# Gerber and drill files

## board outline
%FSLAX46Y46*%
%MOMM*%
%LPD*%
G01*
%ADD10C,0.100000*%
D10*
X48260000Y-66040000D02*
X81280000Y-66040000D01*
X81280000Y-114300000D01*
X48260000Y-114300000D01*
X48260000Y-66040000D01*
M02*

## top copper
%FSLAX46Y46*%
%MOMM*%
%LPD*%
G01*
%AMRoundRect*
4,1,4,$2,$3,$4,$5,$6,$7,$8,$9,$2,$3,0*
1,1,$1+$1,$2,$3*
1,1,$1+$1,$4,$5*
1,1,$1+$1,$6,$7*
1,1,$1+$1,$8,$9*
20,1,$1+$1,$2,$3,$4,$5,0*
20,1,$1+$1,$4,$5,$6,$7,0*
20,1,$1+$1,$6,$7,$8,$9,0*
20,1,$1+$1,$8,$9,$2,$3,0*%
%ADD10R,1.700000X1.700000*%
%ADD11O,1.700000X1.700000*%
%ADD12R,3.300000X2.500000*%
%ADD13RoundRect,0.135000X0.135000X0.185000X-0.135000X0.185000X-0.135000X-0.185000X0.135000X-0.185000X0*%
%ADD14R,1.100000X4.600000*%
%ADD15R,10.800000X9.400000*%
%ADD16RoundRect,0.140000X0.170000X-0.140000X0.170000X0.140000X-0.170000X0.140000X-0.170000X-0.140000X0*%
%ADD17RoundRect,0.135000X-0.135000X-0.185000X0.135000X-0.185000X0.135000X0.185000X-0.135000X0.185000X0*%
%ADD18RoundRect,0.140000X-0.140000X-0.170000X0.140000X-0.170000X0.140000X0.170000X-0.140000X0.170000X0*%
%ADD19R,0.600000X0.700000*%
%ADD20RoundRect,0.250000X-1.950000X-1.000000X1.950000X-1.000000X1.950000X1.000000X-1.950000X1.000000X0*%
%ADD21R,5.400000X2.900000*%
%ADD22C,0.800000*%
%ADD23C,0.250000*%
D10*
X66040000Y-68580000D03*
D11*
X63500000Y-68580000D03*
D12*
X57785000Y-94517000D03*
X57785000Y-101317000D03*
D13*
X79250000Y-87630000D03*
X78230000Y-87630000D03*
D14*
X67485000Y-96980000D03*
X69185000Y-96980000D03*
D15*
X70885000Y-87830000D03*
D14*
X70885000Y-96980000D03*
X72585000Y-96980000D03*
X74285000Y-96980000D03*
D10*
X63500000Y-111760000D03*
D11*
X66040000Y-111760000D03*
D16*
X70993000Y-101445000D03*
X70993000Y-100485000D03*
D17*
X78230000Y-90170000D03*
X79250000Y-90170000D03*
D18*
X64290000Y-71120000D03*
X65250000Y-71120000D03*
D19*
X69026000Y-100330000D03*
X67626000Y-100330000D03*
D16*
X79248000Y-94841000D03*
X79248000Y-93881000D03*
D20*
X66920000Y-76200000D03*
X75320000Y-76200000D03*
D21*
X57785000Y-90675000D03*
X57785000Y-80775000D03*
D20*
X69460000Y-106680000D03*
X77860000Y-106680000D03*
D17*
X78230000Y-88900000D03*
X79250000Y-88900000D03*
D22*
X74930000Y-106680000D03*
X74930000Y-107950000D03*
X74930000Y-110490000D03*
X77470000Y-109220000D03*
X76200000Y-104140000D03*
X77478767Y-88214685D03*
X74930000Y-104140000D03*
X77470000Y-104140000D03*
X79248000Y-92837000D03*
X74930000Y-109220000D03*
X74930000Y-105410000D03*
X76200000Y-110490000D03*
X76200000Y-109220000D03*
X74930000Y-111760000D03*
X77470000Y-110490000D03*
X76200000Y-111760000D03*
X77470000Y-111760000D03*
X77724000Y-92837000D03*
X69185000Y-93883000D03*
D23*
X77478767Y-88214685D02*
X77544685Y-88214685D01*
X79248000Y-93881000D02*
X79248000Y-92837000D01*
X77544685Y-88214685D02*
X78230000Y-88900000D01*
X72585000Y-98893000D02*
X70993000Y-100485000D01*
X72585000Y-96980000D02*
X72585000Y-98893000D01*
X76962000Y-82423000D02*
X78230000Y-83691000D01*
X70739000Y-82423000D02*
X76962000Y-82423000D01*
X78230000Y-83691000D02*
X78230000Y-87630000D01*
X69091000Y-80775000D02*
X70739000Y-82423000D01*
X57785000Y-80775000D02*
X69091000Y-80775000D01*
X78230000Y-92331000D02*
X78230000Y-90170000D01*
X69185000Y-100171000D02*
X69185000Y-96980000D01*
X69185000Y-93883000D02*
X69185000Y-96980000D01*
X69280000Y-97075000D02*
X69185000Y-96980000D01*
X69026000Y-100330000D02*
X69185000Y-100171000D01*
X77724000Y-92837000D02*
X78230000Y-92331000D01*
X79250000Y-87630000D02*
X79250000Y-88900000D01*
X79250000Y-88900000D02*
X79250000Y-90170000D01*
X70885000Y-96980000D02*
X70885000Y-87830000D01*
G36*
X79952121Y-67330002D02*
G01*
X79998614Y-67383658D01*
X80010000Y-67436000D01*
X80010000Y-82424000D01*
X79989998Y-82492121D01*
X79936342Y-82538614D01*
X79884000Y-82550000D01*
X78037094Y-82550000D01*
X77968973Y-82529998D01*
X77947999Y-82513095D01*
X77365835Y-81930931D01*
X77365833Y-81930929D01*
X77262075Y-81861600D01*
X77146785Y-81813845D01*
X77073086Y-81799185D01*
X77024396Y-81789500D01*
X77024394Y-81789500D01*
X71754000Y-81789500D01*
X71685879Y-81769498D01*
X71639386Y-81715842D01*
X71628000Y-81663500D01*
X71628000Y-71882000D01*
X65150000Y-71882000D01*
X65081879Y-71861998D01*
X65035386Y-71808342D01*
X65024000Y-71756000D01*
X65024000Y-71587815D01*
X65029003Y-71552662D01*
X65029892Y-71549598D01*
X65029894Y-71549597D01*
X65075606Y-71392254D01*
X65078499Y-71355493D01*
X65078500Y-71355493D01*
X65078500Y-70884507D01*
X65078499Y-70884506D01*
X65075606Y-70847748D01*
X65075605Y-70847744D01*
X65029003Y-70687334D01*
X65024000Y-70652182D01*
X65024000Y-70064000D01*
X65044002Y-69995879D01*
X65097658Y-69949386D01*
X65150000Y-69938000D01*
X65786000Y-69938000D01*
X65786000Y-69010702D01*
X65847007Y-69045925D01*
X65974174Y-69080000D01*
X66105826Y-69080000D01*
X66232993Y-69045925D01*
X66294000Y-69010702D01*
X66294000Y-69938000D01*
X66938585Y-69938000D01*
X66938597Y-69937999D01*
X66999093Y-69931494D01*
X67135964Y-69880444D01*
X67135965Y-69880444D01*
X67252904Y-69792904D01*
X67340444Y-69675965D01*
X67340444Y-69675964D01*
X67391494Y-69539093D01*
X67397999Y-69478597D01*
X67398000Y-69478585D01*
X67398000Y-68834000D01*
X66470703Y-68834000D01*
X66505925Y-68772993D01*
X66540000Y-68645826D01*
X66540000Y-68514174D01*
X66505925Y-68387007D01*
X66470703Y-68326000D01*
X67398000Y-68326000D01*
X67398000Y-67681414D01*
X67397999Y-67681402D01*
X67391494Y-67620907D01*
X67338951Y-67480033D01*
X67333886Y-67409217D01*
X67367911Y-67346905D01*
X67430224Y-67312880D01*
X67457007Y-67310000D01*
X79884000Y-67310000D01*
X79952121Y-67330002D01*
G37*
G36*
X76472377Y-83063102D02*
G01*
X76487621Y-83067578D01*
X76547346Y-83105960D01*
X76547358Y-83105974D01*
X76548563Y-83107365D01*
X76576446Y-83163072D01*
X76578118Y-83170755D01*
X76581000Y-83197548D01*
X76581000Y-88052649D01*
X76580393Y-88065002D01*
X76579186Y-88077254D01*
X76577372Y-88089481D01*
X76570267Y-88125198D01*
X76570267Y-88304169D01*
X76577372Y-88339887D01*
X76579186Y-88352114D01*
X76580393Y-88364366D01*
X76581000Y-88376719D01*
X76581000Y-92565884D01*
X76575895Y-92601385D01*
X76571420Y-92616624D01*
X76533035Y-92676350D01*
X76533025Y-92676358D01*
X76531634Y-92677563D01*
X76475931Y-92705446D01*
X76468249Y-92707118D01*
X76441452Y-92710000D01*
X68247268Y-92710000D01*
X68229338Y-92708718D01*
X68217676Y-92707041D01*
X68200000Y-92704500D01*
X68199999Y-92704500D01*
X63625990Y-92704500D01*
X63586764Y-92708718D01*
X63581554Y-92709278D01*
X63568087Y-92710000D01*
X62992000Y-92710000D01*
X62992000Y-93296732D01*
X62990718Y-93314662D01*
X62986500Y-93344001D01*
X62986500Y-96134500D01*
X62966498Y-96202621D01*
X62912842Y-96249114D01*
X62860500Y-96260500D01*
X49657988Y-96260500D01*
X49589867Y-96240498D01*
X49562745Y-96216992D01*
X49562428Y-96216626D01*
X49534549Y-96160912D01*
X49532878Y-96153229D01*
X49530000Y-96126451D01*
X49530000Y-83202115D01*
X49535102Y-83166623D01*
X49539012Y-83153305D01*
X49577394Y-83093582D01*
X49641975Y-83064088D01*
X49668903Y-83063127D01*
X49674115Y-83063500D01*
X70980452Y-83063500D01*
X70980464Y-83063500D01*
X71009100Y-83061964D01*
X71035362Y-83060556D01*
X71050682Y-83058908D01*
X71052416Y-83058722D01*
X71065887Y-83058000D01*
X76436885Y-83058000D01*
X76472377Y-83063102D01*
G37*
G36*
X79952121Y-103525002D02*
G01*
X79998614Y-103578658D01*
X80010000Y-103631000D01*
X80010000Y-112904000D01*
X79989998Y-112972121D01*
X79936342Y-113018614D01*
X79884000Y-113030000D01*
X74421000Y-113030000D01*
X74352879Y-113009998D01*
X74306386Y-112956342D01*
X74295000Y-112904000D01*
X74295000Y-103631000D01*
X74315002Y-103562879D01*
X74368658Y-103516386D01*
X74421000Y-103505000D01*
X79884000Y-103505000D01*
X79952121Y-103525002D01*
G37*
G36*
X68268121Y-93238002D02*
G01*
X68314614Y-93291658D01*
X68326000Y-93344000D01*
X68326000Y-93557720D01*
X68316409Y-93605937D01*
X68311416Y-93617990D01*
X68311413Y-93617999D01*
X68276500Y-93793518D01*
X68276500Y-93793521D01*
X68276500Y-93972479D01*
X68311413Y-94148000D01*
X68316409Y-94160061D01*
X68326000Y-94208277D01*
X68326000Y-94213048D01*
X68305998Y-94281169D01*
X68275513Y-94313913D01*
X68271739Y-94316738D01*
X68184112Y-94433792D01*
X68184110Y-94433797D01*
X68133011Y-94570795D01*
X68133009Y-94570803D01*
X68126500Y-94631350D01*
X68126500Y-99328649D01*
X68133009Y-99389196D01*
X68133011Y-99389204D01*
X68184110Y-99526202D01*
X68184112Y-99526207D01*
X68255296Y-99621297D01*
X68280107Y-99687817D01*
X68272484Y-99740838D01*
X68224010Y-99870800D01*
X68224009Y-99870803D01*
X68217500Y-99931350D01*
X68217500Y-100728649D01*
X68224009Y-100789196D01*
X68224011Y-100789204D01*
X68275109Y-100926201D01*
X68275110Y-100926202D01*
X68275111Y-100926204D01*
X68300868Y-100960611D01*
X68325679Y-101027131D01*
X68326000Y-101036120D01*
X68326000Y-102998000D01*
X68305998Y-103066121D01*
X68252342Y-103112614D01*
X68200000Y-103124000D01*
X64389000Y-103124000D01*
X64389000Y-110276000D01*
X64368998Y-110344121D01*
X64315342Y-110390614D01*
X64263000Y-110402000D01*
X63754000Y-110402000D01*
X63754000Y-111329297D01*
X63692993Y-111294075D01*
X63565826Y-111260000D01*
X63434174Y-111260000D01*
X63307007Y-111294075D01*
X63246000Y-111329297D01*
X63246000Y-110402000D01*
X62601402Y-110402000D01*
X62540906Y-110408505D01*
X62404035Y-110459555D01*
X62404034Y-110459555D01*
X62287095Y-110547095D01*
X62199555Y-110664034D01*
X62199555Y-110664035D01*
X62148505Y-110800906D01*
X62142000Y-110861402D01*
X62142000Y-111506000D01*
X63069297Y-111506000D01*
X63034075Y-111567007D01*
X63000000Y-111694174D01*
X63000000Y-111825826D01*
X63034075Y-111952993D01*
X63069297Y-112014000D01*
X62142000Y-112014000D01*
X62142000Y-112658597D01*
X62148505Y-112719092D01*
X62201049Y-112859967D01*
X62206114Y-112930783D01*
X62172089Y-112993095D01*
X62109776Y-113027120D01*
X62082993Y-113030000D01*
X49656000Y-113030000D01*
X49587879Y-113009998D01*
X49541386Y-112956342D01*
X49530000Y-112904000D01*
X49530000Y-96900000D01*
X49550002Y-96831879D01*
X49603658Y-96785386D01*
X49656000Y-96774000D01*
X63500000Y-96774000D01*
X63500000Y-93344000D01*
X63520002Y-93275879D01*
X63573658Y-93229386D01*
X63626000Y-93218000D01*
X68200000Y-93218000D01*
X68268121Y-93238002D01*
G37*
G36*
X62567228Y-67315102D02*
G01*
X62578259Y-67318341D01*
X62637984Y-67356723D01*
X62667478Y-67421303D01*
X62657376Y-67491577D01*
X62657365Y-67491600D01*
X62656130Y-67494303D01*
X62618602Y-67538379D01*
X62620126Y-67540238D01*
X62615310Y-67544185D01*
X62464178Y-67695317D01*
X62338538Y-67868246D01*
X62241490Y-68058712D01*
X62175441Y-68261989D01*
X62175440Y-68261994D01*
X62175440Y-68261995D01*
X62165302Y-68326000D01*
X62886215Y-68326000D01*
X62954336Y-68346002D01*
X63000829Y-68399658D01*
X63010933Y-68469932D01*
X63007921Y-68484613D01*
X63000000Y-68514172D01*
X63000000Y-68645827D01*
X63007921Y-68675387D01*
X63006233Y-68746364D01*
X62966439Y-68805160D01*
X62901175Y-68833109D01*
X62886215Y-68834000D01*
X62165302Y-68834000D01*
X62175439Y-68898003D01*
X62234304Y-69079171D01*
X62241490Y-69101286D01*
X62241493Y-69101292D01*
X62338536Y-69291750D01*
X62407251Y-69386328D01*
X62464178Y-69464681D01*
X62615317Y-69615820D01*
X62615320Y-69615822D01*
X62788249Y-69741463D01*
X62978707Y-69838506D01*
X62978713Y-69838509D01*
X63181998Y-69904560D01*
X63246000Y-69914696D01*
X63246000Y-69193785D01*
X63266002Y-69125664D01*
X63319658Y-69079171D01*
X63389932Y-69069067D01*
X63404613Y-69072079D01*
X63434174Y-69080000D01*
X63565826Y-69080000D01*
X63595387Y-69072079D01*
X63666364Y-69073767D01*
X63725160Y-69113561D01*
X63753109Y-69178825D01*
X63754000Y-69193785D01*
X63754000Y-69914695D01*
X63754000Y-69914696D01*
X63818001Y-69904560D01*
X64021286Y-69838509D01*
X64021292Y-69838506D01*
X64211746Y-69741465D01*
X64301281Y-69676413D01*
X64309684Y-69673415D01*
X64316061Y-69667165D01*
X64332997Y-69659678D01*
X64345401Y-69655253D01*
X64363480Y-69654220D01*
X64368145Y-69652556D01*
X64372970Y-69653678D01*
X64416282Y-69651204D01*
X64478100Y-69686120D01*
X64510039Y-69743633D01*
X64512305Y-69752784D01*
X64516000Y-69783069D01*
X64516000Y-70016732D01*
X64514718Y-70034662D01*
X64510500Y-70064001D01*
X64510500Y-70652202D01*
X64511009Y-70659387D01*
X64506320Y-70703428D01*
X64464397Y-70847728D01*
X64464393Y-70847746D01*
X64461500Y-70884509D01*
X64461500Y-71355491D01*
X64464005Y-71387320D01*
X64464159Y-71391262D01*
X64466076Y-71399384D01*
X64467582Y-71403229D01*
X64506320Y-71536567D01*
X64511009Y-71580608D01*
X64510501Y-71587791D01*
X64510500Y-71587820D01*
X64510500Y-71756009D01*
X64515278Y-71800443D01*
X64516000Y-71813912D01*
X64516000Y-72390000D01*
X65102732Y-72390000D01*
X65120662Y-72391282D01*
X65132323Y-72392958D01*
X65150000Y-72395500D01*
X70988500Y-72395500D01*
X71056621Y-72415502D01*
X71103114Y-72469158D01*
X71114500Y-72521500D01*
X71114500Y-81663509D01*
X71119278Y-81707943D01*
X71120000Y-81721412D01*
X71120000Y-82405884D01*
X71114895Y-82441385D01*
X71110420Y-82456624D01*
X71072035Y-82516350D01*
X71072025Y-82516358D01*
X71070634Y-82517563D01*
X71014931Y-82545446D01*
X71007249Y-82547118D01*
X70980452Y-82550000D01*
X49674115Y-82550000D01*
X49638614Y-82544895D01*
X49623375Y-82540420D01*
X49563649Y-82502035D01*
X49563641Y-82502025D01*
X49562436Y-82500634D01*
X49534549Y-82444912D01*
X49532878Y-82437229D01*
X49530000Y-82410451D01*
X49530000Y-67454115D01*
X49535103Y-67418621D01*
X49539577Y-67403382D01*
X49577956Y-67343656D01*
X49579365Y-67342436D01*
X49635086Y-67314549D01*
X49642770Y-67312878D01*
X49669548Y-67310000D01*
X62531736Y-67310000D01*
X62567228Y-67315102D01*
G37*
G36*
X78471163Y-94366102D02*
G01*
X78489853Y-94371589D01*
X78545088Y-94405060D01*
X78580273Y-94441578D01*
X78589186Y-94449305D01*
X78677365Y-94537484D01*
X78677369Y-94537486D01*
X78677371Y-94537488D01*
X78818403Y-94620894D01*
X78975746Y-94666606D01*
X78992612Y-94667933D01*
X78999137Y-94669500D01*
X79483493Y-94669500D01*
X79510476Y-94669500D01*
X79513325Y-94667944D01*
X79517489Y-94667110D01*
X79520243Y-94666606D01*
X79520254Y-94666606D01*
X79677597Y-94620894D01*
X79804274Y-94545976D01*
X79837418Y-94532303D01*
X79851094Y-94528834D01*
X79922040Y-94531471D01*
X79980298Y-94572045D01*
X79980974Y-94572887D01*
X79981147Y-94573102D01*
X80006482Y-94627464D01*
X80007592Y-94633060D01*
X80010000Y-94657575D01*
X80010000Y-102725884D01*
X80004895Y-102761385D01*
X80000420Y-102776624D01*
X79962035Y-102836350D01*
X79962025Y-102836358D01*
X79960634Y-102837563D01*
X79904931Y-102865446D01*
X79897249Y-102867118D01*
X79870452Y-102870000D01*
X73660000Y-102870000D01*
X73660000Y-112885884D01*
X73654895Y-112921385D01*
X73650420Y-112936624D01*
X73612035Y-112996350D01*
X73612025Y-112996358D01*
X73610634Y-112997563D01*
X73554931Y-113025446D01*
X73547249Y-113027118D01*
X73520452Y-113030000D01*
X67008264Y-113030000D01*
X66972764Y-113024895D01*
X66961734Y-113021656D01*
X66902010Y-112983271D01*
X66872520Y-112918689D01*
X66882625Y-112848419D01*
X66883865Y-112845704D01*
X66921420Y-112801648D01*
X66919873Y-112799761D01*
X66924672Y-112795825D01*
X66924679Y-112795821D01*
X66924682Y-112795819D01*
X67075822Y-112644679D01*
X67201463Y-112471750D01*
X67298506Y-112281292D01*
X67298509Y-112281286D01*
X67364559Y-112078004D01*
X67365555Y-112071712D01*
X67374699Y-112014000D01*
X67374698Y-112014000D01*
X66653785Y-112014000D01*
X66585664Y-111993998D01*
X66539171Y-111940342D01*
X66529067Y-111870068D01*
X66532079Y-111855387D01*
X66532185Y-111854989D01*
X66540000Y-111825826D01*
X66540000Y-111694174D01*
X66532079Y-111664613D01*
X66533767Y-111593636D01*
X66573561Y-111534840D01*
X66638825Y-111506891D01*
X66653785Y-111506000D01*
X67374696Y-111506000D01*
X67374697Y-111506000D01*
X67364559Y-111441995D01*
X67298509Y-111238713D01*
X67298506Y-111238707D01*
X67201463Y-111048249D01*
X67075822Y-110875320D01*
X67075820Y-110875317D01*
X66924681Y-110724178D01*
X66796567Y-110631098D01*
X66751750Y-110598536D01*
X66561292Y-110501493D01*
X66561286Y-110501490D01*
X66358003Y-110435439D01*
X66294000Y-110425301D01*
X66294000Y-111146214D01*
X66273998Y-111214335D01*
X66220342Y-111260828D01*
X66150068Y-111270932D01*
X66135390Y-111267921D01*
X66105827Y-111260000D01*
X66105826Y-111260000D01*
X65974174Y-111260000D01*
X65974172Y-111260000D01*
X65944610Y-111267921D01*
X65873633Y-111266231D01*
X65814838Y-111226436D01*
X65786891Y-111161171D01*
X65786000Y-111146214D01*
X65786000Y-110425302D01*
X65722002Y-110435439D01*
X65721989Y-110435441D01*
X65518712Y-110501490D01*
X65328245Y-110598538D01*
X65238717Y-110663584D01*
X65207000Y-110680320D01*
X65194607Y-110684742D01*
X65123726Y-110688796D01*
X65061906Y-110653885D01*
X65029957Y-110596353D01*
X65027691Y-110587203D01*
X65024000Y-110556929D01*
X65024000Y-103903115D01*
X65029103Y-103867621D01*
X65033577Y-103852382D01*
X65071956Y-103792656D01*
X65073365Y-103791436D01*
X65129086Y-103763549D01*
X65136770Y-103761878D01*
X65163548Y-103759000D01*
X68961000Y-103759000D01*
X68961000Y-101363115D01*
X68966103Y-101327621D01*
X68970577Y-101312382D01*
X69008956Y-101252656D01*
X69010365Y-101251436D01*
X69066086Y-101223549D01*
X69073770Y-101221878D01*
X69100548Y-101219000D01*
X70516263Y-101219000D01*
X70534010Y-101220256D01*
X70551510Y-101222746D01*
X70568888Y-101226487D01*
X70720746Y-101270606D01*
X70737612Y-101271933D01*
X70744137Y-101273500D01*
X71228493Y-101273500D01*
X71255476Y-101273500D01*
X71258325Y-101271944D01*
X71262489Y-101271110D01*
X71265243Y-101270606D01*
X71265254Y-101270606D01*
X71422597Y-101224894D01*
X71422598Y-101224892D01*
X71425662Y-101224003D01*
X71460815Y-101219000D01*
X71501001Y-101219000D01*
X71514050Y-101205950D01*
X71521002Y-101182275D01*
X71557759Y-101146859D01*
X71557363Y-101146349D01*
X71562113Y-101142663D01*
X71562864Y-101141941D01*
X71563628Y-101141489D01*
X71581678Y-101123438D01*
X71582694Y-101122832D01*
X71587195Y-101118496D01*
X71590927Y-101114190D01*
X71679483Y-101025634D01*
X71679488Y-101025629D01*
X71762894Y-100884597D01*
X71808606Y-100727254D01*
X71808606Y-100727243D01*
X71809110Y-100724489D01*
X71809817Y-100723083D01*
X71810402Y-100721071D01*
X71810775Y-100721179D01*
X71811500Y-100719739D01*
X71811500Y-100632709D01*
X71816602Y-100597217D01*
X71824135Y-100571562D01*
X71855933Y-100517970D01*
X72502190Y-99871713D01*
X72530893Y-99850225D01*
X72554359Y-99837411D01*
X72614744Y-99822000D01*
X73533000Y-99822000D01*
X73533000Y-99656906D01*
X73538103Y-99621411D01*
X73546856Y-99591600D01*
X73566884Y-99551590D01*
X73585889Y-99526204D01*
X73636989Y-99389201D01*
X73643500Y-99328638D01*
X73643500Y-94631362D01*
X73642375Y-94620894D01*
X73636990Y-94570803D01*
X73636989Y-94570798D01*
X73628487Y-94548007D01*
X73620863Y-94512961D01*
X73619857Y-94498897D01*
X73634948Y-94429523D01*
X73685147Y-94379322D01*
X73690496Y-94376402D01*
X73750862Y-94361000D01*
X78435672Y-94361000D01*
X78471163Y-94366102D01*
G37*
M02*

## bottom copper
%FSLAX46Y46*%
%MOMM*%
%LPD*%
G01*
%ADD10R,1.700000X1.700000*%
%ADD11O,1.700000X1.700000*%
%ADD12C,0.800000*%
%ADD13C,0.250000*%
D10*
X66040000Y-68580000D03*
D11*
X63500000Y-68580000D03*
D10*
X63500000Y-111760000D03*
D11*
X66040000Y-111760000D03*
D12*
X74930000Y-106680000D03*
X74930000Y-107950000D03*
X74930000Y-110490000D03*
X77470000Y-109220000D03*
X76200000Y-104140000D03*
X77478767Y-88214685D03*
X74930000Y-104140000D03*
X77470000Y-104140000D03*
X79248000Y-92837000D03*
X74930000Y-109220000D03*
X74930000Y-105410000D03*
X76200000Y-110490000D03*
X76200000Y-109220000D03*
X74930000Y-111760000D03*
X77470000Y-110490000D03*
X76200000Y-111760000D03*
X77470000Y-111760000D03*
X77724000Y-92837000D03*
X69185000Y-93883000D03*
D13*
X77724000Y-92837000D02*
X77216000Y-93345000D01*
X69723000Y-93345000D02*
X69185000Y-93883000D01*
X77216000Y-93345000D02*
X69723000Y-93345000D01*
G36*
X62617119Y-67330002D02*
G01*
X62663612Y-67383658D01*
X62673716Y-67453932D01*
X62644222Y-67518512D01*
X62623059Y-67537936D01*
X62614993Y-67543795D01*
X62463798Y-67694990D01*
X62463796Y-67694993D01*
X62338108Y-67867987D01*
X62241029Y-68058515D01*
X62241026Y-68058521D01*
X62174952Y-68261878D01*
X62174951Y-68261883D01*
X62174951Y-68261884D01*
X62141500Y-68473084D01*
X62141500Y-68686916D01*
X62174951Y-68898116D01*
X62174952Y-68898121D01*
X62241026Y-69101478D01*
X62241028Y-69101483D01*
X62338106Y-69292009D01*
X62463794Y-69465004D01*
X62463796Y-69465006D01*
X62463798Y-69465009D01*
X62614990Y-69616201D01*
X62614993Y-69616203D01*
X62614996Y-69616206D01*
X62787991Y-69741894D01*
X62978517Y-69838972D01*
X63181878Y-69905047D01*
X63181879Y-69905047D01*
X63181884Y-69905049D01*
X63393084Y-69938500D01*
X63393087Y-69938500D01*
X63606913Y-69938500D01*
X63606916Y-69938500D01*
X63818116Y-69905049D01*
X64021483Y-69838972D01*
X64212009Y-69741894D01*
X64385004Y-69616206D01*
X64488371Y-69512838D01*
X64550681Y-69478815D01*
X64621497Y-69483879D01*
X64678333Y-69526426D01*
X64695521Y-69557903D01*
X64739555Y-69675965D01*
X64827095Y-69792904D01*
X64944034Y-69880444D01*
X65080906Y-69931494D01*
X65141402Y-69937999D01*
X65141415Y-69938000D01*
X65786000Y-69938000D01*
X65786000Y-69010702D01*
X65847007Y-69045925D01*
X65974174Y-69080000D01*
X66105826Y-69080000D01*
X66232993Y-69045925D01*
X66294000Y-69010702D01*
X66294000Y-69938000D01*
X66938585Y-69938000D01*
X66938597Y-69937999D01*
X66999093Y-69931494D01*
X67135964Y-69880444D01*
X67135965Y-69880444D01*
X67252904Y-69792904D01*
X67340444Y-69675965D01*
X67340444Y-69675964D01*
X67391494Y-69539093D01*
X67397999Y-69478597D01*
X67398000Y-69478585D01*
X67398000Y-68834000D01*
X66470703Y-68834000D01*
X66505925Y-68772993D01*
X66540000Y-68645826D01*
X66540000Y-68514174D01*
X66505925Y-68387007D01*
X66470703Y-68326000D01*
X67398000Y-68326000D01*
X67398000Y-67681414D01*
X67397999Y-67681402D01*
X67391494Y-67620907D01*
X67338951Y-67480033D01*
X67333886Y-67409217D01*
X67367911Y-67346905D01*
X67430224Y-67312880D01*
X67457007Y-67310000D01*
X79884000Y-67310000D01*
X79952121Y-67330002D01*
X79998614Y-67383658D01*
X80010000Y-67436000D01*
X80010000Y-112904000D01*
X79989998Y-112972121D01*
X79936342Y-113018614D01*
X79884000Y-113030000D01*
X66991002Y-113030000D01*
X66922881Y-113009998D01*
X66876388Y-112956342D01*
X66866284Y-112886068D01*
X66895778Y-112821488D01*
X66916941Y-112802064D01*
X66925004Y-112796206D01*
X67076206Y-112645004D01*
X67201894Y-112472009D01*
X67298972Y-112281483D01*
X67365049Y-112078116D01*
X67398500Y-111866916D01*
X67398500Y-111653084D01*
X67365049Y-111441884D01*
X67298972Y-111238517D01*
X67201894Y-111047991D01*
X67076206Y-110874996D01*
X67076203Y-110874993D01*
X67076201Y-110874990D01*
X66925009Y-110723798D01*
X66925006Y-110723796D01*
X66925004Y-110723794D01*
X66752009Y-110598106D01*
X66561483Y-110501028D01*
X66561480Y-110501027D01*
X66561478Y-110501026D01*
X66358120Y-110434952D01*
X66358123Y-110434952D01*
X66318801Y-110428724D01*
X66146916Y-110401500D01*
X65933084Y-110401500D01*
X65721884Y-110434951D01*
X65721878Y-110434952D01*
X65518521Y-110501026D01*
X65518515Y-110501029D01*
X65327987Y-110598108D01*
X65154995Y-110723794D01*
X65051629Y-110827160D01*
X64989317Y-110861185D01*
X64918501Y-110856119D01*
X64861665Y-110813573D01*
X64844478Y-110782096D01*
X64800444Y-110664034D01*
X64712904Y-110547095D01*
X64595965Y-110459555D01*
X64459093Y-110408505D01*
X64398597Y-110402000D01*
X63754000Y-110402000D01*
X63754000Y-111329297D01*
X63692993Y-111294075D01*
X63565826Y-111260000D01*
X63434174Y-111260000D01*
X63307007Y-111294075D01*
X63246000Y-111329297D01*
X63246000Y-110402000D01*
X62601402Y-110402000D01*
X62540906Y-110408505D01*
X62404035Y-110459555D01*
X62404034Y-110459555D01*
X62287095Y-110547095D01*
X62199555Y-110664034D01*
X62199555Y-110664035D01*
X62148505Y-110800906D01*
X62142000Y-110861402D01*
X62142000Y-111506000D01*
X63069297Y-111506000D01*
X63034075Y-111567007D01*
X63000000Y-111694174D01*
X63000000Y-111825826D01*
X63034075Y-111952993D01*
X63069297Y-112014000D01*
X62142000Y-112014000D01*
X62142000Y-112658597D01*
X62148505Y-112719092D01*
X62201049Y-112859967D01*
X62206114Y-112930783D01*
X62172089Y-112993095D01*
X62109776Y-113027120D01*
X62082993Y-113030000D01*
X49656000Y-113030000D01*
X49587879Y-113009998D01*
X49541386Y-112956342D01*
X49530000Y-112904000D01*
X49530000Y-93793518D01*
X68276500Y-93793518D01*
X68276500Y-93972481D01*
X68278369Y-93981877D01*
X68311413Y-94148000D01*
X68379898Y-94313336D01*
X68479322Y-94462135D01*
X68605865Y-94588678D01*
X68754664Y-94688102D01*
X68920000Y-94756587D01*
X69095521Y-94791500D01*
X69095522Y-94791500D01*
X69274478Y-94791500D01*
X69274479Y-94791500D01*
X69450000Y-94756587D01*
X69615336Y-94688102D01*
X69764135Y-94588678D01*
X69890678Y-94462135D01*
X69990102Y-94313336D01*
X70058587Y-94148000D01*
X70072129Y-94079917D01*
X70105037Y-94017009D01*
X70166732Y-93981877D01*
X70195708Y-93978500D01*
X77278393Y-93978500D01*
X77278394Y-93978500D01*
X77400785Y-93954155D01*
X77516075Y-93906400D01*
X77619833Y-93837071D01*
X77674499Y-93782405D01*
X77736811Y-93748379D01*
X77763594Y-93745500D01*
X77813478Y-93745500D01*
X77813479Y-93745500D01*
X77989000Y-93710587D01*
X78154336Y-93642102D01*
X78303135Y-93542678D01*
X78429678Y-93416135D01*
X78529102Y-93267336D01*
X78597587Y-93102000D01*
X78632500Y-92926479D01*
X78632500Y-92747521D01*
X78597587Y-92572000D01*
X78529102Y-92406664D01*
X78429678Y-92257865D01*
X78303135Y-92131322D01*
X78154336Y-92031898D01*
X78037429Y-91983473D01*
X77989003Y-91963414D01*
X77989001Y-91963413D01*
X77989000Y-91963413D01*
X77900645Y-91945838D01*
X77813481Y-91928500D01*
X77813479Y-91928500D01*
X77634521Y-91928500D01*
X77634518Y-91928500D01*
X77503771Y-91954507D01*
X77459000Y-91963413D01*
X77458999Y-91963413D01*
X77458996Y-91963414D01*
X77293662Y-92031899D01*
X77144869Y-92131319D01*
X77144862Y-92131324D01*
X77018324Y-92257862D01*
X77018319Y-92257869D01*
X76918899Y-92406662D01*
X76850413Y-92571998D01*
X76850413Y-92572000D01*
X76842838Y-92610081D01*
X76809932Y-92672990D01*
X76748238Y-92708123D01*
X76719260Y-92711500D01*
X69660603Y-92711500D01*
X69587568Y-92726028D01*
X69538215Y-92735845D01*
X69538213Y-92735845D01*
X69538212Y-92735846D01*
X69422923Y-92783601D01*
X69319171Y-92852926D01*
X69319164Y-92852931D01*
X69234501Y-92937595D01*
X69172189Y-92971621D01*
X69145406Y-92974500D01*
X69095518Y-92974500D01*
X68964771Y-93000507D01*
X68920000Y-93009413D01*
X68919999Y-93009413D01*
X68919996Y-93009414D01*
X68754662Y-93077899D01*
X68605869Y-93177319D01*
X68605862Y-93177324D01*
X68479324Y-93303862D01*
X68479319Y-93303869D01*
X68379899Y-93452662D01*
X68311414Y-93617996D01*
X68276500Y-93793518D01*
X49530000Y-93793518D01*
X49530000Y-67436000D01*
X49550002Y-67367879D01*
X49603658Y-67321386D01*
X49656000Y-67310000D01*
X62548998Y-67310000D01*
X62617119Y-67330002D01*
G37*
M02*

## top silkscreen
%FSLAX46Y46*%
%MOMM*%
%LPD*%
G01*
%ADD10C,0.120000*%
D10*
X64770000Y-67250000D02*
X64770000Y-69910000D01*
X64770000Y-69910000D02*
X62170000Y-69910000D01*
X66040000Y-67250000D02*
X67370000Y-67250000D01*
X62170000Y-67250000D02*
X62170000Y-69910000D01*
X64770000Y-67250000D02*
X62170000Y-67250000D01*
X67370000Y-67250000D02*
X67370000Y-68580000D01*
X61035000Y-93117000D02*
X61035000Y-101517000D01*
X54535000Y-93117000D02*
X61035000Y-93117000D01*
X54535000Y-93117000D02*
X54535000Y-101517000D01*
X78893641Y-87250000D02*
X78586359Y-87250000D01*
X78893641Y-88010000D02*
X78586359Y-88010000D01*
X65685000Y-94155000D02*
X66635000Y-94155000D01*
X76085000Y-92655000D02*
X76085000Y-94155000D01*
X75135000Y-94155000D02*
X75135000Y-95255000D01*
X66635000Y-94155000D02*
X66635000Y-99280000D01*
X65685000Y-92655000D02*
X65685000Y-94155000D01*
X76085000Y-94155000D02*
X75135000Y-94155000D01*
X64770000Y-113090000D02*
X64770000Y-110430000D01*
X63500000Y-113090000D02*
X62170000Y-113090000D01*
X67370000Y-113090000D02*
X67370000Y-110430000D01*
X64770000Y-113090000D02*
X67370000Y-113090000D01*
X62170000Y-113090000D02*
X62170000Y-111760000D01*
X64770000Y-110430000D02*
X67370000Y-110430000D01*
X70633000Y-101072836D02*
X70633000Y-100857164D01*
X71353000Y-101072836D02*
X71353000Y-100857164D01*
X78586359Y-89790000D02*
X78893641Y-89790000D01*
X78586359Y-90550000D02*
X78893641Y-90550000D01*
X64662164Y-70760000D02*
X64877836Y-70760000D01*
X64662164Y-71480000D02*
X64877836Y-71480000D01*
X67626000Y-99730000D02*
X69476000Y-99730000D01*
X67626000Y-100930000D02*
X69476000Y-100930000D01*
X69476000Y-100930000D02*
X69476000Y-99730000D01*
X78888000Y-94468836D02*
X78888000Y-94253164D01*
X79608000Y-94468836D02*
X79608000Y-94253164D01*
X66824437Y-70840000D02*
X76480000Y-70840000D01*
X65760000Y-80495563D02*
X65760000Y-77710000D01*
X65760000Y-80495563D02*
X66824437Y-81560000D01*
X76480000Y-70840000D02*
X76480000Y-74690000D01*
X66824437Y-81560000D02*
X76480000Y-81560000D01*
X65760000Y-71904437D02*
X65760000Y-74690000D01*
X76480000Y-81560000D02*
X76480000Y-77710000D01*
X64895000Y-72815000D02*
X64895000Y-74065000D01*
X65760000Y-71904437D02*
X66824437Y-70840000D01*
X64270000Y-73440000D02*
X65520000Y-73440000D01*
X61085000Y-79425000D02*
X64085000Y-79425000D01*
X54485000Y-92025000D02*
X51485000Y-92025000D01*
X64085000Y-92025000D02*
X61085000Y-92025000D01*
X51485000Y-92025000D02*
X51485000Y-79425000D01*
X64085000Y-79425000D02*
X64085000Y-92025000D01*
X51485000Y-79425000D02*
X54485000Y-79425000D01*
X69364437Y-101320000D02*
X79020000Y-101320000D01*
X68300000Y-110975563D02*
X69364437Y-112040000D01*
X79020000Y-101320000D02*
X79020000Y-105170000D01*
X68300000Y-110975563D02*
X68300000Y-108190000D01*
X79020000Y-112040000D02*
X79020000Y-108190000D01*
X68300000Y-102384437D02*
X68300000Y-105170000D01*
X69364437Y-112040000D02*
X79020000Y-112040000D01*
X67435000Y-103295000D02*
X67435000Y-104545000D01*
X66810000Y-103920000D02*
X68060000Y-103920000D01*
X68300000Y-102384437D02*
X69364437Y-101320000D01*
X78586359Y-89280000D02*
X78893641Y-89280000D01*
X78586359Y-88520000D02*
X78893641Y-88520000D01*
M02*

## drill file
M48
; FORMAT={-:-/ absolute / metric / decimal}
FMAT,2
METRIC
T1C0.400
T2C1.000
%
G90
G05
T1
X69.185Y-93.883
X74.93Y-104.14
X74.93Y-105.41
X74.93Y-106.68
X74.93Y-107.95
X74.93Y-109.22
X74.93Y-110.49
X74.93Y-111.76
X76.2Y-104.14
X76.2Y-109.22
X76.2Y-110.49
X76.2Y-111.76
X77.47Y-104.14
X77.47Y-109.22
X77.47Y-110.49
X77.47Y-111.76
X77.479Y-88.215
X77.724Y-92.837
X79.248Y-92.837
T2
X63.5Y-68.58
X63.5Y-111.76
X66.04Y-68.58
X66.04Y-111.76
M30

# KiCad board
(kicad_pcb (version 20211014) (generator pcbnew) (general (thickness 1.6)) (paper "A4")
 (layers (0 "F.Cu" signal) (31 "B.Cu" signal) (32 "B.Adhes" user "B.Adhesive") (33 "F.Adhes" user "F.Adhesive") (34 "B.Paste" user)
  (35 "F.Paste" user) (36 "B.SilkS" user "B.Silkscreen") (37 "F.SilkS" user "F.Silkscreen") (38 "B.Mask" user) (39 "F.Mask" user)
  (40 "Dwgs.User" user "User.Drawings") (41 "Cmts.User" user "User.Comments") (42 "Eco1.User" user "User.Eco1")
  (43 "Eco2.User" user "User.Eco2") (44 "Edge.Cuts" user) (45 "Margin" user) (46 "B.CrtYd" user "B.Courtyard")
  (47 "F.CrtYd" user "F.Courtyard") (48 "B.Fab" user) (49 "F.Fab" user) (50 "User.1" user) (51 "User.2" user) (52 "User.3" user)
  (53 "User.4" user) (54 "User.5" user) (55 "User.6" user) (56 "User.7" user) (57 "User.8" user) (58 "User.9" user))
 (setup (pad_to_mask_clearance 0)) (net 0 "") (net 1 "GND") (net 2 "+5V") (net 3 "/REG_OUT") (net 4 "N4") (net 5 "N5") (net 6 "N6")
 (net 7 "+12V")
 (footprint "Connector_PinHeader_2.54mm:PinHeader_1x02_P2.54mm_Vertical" (layer "F.Cu") (at 66.04 68.58 -90)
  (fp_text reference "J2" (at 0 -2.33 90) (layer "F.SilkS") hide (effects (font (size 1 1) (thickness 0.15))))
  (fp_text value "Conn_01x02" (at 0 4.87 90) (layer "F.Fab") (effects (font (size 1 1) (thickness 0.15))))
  (fp_line (start -1.33 1.27) (end 1.33 1.27) (layer "F.SilkS") (width 0.12))
  (fp_line (start 1.33 1.27) (end 1.33 3.87) (layer "F.SilkS") (width 0.12))
  (fp_line (start -1.33 0) (end -1.33 -1.33) (layer "F.SilkS") (width 0.12))
  (fp_line (start -1.33 3.87) (end 1.33 3.87) (layer "F.SilkS") (width 0.12))
  (fp_line (start -1.33 1.27) (end -1.33 3.87) (layer "F.SilkS") (width 0.12))
  (fp_line (start -1.33 -1.33) (end 0 -1.33) (layer "F.SilkS") (width 0.12))
  (pad "1" thru_hole rect (at 0 0 270) (size 1.7 1.7) (drill 1) (layers *.Cu *.Mask) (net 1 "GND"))
  (pad "2" thru_hole oval (at 0 2.54 270) (size 1.7 1.7) (drill 1) (layers *.Cu *.Mask) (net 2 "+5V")))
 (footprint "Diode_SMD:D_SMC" (layer "F.Cu") (at 57.785 97.917 -90)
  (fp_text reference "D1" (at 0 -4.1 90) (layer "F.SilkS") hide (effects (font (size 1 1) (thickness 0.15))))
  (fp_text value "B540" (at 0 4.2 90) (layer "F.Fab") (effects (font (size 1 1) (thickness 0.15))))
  (fp_line (start -4.8 -3.25) (end 3.6 -3.25) (layer "F.SilkS") (width 0.12))
  (fp_line (start -4.8 3.25) (end -4.8 -3.25) (layer "F.SilkS") (width 0.12))
  (fp_line (start -4.8 3.25) (end 3.6 3.25) (layer "F.SilkS") (width 0.12))
  (pad "1" smd rect (at -3.4 0) (size 3.3 2.5) (layers "F.Cu" "F.Paste" "F.Mask") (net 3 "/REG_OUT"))
  (pad "2" smd rect (at 3.4 0) (size 3.3 2.5) (layers "F.Cu" "F.Paste" "F.Mask") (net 1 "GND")))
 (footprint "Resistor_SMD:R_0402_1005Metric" (layer "F.Cu") (at 78.74 87.63 180)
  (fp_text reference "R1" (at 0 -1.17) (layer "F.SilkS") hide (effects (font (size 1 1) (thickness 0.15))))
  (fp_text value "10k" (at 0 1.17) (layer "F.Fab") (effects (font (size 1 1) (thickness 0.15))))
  (fp_line (start -0.153641 0.38) (end 0.153641 0.38) (layer "F.SilkS") (width 0.12))
  (fp_line (start -0.153641 -0.38) (end 0.153641 -0.38) (layer "F.SilkS") (width 0.12))
  (pad "1" smd roundrect (at -0.51 0 180) (size 0.54 0.64) (layers "F.Cu" "F.Paste" "F.Mask") (roundrect_rratio 0.25) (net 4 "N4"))
  (pad "2" smd roundrect (at 0.51 0 180) (size 0.54 0.64) (layers "F.Cu" "F.Paste" "F.Mask") (roundrect_rratio 0.25) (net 2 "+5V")))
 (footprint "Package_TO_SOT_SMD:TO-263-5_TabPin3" (layer "F.Cu") (at 70.885 91.205 90)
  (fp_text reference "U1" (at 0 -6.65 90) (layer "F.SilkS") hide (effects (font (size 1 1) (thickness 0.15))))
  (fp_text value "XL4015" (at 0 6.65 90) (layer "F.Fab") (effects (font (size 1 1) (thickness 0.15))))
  (fp_line (start -2.95 -5.2) (end -2.95 -4.25) (layer "F.SilkS") (width 0.12))
  (fp_line (start -1.45 5.2) (end -2.95 5.2) (layer "F.SilkS") (width 0.12))
  (fp_line (start -2.95 4.25) (end -4.05 4.25) (layer "F.SilkS") (width 0.12))
  (fp_line (start -2.95 -4.25) (end -8.075 -4.25) (layer "F.SilkS") (width 0.12))
  (fp_line (start -1.45 -5.2) (end -2.95 -5.2) (layer "F.SilkS") (width 0.12))
  (fp_line (start -2.95 5.2) (end -2.95 4.25) (layer "F.SilkS") (width 0.12))
  (pad "" smd rect (at 5.8 2.775 90) (size 4.55 5.25) (layers "F.Paste"))
  (pad "" smd rect (at 0.95 -2.775 90) (size 4.55 5.25) (layers "F.Paste"))
  (pad "" smd rect (at 5.8 -2.775 90) (size 4.55 5.25) (layers "F.Paste"))
  (pad "" smd rect (at 0.95 2.775 90) (size 4.55 5.25) (layers "F.Paste"))
  (pad "1" smd rect (at -5.775 -3.4 90) (size 4.6 1.1) (layers "F.Cu" "F.Paste" "F.Mask") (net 1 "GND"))
  (pad "2" smd rect (at -5.775 -1.7 90) (size 4.6 1.1) (layers "F.Cu" "F.Paste" "F.Mask") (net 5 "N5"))
  (pad "3" smd rect (at 3.375 0 90) (size 9.4 10.8) (layers "F.Cu" "F.Mask") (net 3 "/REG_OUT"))
  (pad "3" smd rect (at -5.775 0 90) (size 4.6 1.1) (layers "F.Cu" "F.Paste" "F.Mask") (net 3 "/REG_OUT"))
  (pad "4" smd rect (at -5.775 1.7 90) (size 4.6 1.1) (layers "F.Cu" "F.Paste" "F.Mask") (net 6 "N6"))
  (pad "5" smd rect (at -5.775 3.4 90) (size 4.6 1.1) (layers "F.Cu" "F.Paste" "F.Mask") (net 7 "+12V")))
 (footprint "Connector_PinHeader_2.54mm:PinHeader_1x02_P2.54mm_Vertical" (layer "F.Cu") (at 63.5 111.76 90)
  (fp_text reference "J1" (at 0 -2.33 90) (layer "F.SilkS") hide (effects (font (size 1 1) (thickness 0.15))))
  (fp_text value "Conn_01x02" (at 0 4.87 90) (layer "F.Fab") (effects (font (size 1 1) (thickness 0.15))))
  (fp_line (start -1.33 1.27) (end 1.33 1.27) (layer "F.SilkS") (width 0.12))
  (fp_line (start -1.33 0) (end -1.33 -1.33) (layer "F.SilkS") (width 0.12))
  (fp_line (start -1.33 3.87) (end 1.33 3.87) (layer "F.SilkS") (width 0.12))
  (fp_line (start -1.33 1.27) (end -1.33 3.87) (layer "F.SilkS") (width 0.12))
  (fp_line (start -1.33 -1.33) (end 0 -1.33) (layer "F.SilkS") (width 0.12))
  (fp_line (start 1.33 1.27) (end 1.33 3.87) (layer "F.SilkS") (width 0.12))
  (pad "1" thru_hole rect (at 0 0 90) (size 1.7 1.7) (drill 1) (layers *.Cu *.Mask) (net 1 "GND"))
  (pad "2" thru_hole oval (at 0 2.54 90) (size 1.7 1.7) (drill 1) (layers *.Cu *.Mask) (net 7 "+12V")))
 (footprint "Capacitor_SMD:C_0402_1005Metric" (layer "F.Cu") (at 70.993 100.965 90)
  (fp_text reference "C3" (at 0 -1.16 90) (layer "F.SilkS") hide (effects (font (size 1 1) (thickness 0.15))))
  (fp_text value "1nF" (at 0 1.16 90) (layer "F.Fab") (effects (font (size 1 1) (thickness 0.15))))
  (fp_line (start -0.107836 -0.36) (end 0.107836 -0.36) (layer "F.SilkS") (width 0.12))
  (fp_line (start -0.107836 0.36) (end 0.107836 0.36) (layer "F.SilkS") (width 0.12))
  (pad "1" smd roundrect (at -0.48 0 90) (size 0.56 0.62) (layers "F.Cu" "F.Paste" "F.Mask") (roundrect_rratio 0.25) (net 7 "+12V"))
  (pad "2" smd roundrect (at 0.48 0 90) (size 0.56 0.62) (layers "F.Cu" "F.Paste" "F.Mask") (roundrect_rratio 0.25) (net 6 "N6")))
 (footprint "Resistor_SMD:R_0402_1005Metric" (layer "F.Cu") (at 78.74 90.17)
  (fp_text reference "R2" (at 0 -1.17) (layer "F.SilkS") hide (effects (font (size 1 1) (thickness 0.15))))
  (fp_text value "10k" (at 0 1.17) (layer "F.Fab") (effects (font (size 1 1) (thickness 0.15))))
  (fp_line (start -0.153641 -0.38) (end 0.153641 -0.38) (layer "F.SilkS") (width 0.12))
  (fp_line (start -0.153641 0.38) (end 0.153641 0.38) (layer "F.SilkS") (width 0.12))
  (pad "1" smd roundrect (at -0.51 0) (size 0.54 0.64) (layers "F.Cu" "F.Paste" "F.Mask") (roundrect_rratio 0.25) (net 5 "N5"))
  (pad "2" smd roundrect (at 0.51 0) (size 0.54 0.64) (layers "F.Cu" "F.Paste" "F.Mask") (roundrect_rratio 0.25) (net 4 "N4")))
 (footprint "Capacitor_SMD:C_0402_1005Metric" (layer "F.Cu") (at 64.77 71.12)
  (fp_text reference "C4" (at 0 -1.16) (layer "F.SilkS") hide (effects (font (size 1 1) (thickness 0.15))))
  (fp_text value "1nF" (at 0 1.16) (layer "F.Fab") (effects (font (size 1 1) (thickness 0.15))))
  (fp_line (start -0.107836 -0.36) (end 0.107836 -0.36) (layer "F.SilkS") (width 0.12))
  (fp_line (start -0.107836 0.36) (end 0.107836 0.36) (layer "F.SilkS") (width 0.12))
  (pad "1" smd roundrect (at -0.48 0) (size 0.56 0.62) (layers "F.Cu" "F.Paste" "F.Mask") (roundrect_rratio 0.25) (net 2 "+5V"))
  (pad "2" smd roundrect (at 0.48 0) (size 0.56 0.62) (layers "F.Cu" "F.Paste" "F.Mask") (roundrect_rratio 0.25) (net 1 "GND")))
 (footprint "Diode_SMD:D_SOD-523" (layer "F.Cu") (at 68.326 100.33 180)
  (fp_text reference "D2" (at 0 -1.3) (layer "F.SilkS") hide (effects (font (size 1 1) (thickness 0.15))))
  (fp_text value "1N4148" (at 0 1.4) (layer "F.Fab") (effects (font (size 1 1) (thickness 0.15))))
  (fp_line (start 0.7 0.6) (end -1.15 0.6) (layer "F.SilkS") (width 0.12))
  (fp_line (start 0.7 -0.6) (end -1.15 -0.6) (layer "F.SilkS") (width 0.12))
  (fp_line (start -1.15 -0.6) (end -1.15 0.6) (layer "F.SilkS") (width 0.12))
  (pad "1" smd rect (at -0.7 0) (size 0.6 0.7) (layers "F.Cu" "F.Paste" "F.Mask") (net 5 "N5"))
  (pad "2" smd rect (at 0.7 0) (size 0.6 0.7) (layers "F.Cu" "F.Paste" "F.Mask") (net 1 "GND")))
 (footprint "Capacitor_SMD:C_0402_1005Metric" (layer "F.Cu") (at 79.248 94.361 90)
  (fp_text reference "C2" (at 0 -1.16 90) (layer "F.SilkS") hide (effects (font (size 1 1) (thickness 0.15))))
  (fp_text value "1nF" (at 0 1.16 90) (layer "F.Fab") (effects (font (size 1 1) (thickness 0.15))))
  (fp_line (start -0.107836 -0.36) (end 0.107836 -0.36) (layer "F.SilkS") (width 0.12))
  (fp_line (start -0.107836 0.36) (end 0.107836 0.36) (layer "F.SilkS") (width 0.12))
  (pad "1" smd roundrect (at -0.48 0 90) (size 0.56 0.62) (layers "F.Cu" "F.Paste" "F.Mask") (roundrect_rratio 0.25) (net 7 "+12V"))
  (pad "2" smd roundrect (at 0.48 0 90) (size 0.56 0.62) (layers "F.Cu" "F.Paste" "F.Mask") (roundrect_rratio 0.25) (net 1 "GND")))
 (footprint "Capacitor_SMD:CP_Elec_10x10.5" (layer "F.Cu") (at 71.12 76.2)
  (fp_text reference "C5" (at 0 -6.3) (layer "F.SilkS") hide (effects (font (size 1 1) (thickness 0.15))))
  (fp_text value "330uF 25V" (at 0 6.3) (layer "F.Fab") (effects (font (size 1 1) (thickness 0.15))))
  (fp_line (start -4.295563 -5.36) (end 5.36 -5.36) (layer "F.SilkS") (width 0.12))
  (fp_line (start -5.36 4.295563) (end -5.36 1.51) (layer "F.SilkS") (width 0.12))
  (fp_line (start -5.36 4.295563) (end -4.295563 5.36) (layer "F.SilkS") (width 0.12))
  (fp_line (start 5.36 -5.36) (end 5.36 -1.51) (layer "F.SilkS") (width 0.12))
  (fp_line (start -4.295563 5.36) (end 5.36 5.36) (layer "F.SilkS") (width 0.12))
  (fp_line (start -5.36 -4.295563) (end -5.36 -1.51) (layer "F.SilkS") (width 0.12))
  (fp_line (start 5.36 5.36) (end 5.36 1.51) (layer "F.SilkS") (width 0.12))
  (fp_line (start -6.225 -3.385) (end -6.225 -2.135) (layer "F.SilkS") (width 0.12))
  (fp_line (start -5.36 -4.295563) (end -4.295563 -5.36) (layer "F.SilkS") (width 0.12))
  (fp_line (start -6.85 -2.76) (end -5.6 -2.76) (layer "F.SilkS") (width 0.12))
  (pad "1" smd roundrect (at -4.2 0) (size 4.4 2.5) (layers "F.Cu" "F.Paste" "F.Mask") (roundrect_rratio 0.1) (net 2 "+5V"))
  (pad "2" smd roundrect (at 4.2 0) (size 4.4 2.5) (layers "F.Cu" "F.Paste" "F.Mask") (roundrect_rratio 0.1) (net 1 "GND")))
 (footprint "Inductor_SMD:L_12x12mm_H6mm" (layer "F.Cu") (at 57.785 85.725 90)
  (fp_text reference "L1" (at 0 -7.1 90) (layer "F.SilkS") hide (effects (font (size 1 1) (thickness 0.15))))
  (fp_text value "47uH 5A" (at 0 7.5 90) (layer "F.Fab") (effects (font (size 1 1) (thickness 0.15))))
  (fp_line (start 6.3 3.3) (end 6.3 6.3) (layer "F.SilkS") (width 0.12))
  (fp_line (start -6.3 -3.3) (end -6.3 -6.3) (layer "F.SilkS") (width 0.12))
  (fp_line (start -6.3 6.3) (end -6.3 3.3) (layer "F.SilkS") (width 0.12))
  (fp_line (start -6.3 -6.3) (end 6.3 -6.3) (layer "F.SilkS") (width 0.12))
  (fp_line (start 6.3 6.3) (end -6.3 6.3) (layer "F.SilkS") (width 0.12))
  (fp_line (start 6.3 -6.3) (end 6.3 -3.3) (layer "F.SilkS") (width 0.12))
  (pad "1" smd rect (at -4.95 0 90) (size 2.9 5.4) (layers "F.Cu" "F.Paste" "F.Mask") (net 3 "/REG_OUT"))
  (pad "2" smd rect (at 4.95 0 90) (size 2.9 5.4) (layers "F.Cu" "F.Paste" "F.Mask") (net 2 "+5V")))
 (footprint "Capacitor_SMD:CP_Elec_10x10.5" (layer "F.Cu") (at 73.66 106.68)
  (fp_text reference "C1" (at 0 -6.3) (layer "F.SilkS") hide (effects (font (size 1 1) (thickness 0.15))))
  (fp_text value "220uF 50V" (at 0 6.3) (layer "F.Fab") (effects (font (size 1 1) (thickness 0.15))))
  (fp_line (start -4.295563 -5.36) (end 5.36 -5.36) (layer "F.SilkS") (width 0.12))
  (fp_line (start -5.36 4.295563) (end -4.295563 5.36) (layer "F.SilkS") (width 0.12))
  (fp_line (start 5.36 -5.36) (end 5.36 -1.51) (layer "F.SilkS") (width 0.12))
  (fp_line (start -5.36 4.295563) (end -5.36 1.51) (layer "F.SilkS") (width 0.12))
  (fp_line (start 5.36 5.36) (end 5.36 1.51) (layer "F.SilkS") (width 0.12))
  (fp_line (start -5.36 -4.295563) (end -5.36 -1.51) (layer "F.SilkS") (width 0.12))
  (fp_line (start -4.295563 5.36) (end 5.36 5.36) (layer "F.SilkS") (width 0.12))
  (fp_line (start -6.225 -3.385) (end -6.225 -2.135) (layer "F.SilkS") (width 0.12))
  (fp_line (start -6.85 -2.76) (end -5.6 -2.76) (layer "F.SilkS") (width 0.12))
  (fp_line (start -5.36 -4.295563) (end -4.295563 -5.36) (layer "F.SilkS") (width 0.12))
  (pad "1" smd roundrect (at -4.2 0) (size 4.4 2.5) (layers "F.Cu" "F.Paste" "F.Mask") (roundrect_rratio 0.1) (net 7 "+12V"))
  (pad "2" smd roundrect (at 4.2 0) (size 4.4 2.5) (layers "F.Cu" "F.Paste" "F.Mask") (roundrect_rratio 0.1) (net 1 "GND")))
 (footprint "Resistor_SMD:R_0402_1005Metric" (layer "F.Cu") (at 78.74 88.9)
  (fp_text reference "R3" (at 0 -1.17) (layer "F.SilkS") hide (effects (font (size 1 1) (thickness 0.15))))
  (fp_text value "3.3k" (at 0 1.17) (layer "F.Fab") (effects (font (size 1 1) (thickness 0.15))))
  (fp_line (start -0.153641 0.38) (end 0.153641 0.38) (layer "F.SilkS") (width 0.12))
  (fp_line (start -0.153641 -0.38) (end 0.153641 -0.38) (layer "F.SilkS") (width 0.12))
  (pad "1" smd roundrect (at -0.51 0) (size 0.54 0.64) (layers "F.Cu" "F.Paste" "F.Mask") (roundrect_rratio 0.25) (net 1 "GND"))
  (pad "2" smd roundrect (at 0.51 0) (size 0.54 0.64) (layers "F.Cu" "F.Paste" "F.Mask") (roundrect_rratio 0.25) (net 4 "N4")))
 (gr_rect (start 48.26 66.04) (end 81.28 114.3) (layer "Edge.Cuts") (width 0.1) (fill none))
 (segment (start 77.478767 88.214685) (end 77.544685 88.214685) (width 0.25) (layer "F.Cu") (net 1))
 (segment (start 79.248 93.881) (end 79.248 92.837) (width 0.25) (layer "F.Cu") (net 1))
 (segment (start 77.544685 88.214685) (end 78.23 88.9) (width 0.25) (layer "F.Cu") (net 1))
 (via (at 74.93 106.68) (size 0.8) (drill 0.4) (layers "F.Cu" "B.Cu") (free) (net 1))
 (via (at 74.93 107.95) (size 0.8) (drill 0.4) (layers "F.Cu" "B.Cu") (free) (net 1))
 (via (at 74.93 110.49) (size 0.8) (drill 0.4) (layers "F.Cu" "B.Cu") (free) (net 1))
 (via (at 77.47 109.22) (size 0.8) (drill 0.4) (layers "F.Cu" "B.Cu") (free) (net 1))
 (via (at 76.2 104.14) (size 0.8) (drill 0.4) (layers "F.Cu" "B.Cu") (free) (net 1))
 (via (at 77.478767 88.214685) (size 0.8) (drill 0.4) (layers "F.Cu" "B.Cu") (free) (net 1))
 (via (at 74.93 104.14) (size 0.8) (drill 0.4) (layers "F.Cu" "B.Cu") (free) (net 1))
 (via (at 77.47 104.14) (size 0.8) (drill 0.4) (layers "F.Cu" "B.Cu") (free) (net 1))
 (via (at 79.248 92.837) (size 0.8) (drill 0.4) (layers "F.Cu" "B.Cu") (free) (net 1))
 (via (at 74.93 109.22) (size 0.8) (drill 0.4) (layers "F.Cu" "B.Cu") (free) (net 1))
 (via (at 74.93 105.41) (size 0.8) (drill 0.4) (layers "F.Cu" "B.Cu") (free) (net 1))
 (via (at 76.2 110.49) (size 0.8) (drill 0.4) (layers "F.Cu" "B.Cu") (free) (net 1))
 (via (at 76.2 109.22) (size 0.8) (drill 0.4) (layers "F.Cu" "B.Cu") (free) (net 1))
 (via (at 74.93 111.76) (size 0.8) (drill 0.4) (layers "F.Cu" "B.Cu") (free) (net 1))
 (via (at 77.47 110.49) (size 0.8) (drill 0.4) (layers "F.Cu" "B.Cu") (free) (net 1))
 (via (at 76.2 111.76) (size 0.8) (drill 0.4) (layers "F.Cu" "B.Cu") (free) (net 1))
 (via (at 77.47 111.76) (size 0.8) (drill 0.4) (layers "F.Cu" "B.Cu") (free) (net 1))
 (segment (start 72.585 98.893) (end 70.993 100.485) (width 0.25) (layer "F.Cu") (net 6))
 (segment (start 72.585 96.98) (end 72.585 98.893) (width 0.25) (layer "F.Cu") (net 6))
 (segment (start 76.962 82.423) (end 78.23 83.691) (width 0.25) (layer "F.Cu") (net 2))
 (segment (start 70.739 82.423) (end 76.962 82.423) (width 0.25) (layer "F.Cu") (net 2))
 (segment (start 78.23 83.691) (end 78.23 87.63) (width 0.25) (layer "F.Cu") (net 2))
 (segment (start 69.091 80.775) (end 70.739 82.423) (width 0.25) (layer "F.Cu") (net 2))
 (segment (start 57.785 80.775) (end 69.091 80.775) (width 0.25) (layer "F.Cu") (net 2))
 (segment (start 78.23 92.331) (end 78.23 90.17) (width 0.25) (layer "F.Cu") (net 5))
 (segment (start 69.185 100.171) (end 69.185 96.98) (width 0.25) (layer "F.Cu") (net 5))
 (segment (start 69.185 93.883) (end 69.185 96.98) (width 0.25) (layer "F.Cu") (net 5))
 (segment (start 69.28 97.075) (end 69.185 96.98) (width 0.25) (layer "F.Cu") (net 5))
 (segment (start 69.026 100.33) (end 69.185 100.171) (width 0.25) (layer "F.Cu") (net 5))
 (segment (start 77.724 92.837) (end 78.23 92.331) (width 0.25) (layer "F.Cu") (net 5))
 (via (at 77.724 92.837) (size 0.8) (drill 0.4) (layers "F.Cu" "B.Cu") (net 5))
 (via (at 69.185 93.883) (size 0.8) (drill 0.4) (layers "F.Cu" "B.Cu") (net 5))
 (segment (start 77.724 92.837) (end 77.216 93.345) (width 0.25) (layer "B.Cu") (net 5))
 (segment (start 69.723 93.345) (end 69.185 93.883) (width 0.25) (layer "B.Cu") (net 5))
 (segment (start 77.216 93.345) (end 69.723 93.345) (width 0.25) (layer "B.Cu") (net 5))
 (segment (start 79.25 87.63) (end 79.25 88.9) (width 0.25) (layer "F.Cu") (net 4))
 (segment (start 79.25 88.9) (end 79.25 90.17) (width 0.25) (layer "F.Cu") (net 4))
 (segment (start 70.885 96.98) (end 70.885 87.83) (width 0.25) (layer "F.Cu") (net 3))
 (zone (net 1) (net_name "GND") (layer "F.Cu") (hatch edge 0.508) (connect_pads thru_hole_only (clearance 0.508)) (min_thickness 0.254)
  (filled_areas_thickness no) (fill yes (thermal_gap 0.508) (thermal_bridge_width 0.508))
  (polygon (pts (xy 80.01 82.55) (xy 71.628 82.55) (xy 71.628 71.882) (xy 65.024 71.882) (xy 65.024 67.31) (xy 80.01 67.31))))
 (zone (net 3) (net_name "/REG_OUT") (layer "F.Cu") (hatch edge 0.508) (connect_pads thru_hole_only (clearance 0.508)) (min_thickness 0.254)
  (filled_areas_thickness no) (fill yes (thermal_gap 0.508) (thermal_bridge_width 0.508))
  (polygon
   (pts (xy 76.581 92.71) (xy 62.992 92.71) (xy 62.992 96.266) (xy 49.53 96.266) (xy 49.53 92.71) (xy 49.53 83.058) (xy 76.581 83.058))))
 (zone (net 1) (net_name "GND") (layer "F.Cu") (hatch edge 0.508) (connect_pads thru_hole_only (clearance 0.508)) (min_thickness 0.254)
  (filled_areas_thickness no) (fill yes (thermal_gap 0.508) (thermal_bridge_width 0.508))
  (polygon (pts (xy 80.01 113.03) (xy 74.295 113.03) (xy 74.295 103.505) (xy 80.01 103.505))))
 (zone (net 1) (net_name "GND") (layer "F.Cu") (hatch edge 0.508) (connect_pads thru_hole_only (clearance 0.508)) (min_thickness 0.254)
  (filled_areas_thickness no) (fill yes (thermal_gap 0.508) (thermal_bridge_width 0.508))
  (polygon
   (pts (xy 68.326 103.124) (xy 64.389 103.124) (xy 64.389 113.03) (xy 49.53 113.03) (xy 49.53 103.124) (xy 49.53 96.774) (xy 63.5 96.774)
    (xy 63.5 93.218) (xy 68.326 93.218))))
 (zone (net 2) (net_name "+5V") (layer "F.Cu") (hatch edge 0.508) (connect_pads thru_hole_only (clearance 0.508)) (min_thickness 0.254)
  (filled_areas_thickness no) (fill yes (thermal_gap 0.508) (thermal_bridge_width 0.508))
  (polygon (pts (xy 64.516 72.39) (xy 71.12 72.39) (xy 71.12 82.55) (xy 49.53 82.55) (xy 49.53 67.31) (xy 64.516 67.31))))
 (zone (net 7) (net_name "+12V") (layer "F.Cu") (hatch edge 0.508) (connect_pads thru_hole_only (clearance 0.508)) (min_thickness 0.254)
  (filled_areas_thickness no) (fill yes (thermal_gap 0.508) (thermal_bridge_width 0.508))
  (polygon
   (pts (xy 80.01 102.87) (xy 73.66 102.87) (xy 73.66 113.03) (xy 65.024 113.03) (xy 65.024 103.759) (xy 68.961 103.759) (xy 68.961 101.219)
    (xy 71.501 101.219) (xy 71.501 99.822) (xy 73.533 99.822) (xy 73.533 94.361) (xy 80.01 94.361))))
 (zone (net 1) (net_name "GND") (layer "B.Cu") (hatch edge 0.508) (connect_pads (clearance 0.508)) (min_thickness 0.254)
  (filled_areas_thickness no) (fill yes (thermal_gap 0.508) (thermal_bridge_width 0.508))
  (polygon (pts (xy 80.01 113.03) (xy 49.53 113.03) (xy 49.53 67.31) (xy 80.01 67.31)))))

